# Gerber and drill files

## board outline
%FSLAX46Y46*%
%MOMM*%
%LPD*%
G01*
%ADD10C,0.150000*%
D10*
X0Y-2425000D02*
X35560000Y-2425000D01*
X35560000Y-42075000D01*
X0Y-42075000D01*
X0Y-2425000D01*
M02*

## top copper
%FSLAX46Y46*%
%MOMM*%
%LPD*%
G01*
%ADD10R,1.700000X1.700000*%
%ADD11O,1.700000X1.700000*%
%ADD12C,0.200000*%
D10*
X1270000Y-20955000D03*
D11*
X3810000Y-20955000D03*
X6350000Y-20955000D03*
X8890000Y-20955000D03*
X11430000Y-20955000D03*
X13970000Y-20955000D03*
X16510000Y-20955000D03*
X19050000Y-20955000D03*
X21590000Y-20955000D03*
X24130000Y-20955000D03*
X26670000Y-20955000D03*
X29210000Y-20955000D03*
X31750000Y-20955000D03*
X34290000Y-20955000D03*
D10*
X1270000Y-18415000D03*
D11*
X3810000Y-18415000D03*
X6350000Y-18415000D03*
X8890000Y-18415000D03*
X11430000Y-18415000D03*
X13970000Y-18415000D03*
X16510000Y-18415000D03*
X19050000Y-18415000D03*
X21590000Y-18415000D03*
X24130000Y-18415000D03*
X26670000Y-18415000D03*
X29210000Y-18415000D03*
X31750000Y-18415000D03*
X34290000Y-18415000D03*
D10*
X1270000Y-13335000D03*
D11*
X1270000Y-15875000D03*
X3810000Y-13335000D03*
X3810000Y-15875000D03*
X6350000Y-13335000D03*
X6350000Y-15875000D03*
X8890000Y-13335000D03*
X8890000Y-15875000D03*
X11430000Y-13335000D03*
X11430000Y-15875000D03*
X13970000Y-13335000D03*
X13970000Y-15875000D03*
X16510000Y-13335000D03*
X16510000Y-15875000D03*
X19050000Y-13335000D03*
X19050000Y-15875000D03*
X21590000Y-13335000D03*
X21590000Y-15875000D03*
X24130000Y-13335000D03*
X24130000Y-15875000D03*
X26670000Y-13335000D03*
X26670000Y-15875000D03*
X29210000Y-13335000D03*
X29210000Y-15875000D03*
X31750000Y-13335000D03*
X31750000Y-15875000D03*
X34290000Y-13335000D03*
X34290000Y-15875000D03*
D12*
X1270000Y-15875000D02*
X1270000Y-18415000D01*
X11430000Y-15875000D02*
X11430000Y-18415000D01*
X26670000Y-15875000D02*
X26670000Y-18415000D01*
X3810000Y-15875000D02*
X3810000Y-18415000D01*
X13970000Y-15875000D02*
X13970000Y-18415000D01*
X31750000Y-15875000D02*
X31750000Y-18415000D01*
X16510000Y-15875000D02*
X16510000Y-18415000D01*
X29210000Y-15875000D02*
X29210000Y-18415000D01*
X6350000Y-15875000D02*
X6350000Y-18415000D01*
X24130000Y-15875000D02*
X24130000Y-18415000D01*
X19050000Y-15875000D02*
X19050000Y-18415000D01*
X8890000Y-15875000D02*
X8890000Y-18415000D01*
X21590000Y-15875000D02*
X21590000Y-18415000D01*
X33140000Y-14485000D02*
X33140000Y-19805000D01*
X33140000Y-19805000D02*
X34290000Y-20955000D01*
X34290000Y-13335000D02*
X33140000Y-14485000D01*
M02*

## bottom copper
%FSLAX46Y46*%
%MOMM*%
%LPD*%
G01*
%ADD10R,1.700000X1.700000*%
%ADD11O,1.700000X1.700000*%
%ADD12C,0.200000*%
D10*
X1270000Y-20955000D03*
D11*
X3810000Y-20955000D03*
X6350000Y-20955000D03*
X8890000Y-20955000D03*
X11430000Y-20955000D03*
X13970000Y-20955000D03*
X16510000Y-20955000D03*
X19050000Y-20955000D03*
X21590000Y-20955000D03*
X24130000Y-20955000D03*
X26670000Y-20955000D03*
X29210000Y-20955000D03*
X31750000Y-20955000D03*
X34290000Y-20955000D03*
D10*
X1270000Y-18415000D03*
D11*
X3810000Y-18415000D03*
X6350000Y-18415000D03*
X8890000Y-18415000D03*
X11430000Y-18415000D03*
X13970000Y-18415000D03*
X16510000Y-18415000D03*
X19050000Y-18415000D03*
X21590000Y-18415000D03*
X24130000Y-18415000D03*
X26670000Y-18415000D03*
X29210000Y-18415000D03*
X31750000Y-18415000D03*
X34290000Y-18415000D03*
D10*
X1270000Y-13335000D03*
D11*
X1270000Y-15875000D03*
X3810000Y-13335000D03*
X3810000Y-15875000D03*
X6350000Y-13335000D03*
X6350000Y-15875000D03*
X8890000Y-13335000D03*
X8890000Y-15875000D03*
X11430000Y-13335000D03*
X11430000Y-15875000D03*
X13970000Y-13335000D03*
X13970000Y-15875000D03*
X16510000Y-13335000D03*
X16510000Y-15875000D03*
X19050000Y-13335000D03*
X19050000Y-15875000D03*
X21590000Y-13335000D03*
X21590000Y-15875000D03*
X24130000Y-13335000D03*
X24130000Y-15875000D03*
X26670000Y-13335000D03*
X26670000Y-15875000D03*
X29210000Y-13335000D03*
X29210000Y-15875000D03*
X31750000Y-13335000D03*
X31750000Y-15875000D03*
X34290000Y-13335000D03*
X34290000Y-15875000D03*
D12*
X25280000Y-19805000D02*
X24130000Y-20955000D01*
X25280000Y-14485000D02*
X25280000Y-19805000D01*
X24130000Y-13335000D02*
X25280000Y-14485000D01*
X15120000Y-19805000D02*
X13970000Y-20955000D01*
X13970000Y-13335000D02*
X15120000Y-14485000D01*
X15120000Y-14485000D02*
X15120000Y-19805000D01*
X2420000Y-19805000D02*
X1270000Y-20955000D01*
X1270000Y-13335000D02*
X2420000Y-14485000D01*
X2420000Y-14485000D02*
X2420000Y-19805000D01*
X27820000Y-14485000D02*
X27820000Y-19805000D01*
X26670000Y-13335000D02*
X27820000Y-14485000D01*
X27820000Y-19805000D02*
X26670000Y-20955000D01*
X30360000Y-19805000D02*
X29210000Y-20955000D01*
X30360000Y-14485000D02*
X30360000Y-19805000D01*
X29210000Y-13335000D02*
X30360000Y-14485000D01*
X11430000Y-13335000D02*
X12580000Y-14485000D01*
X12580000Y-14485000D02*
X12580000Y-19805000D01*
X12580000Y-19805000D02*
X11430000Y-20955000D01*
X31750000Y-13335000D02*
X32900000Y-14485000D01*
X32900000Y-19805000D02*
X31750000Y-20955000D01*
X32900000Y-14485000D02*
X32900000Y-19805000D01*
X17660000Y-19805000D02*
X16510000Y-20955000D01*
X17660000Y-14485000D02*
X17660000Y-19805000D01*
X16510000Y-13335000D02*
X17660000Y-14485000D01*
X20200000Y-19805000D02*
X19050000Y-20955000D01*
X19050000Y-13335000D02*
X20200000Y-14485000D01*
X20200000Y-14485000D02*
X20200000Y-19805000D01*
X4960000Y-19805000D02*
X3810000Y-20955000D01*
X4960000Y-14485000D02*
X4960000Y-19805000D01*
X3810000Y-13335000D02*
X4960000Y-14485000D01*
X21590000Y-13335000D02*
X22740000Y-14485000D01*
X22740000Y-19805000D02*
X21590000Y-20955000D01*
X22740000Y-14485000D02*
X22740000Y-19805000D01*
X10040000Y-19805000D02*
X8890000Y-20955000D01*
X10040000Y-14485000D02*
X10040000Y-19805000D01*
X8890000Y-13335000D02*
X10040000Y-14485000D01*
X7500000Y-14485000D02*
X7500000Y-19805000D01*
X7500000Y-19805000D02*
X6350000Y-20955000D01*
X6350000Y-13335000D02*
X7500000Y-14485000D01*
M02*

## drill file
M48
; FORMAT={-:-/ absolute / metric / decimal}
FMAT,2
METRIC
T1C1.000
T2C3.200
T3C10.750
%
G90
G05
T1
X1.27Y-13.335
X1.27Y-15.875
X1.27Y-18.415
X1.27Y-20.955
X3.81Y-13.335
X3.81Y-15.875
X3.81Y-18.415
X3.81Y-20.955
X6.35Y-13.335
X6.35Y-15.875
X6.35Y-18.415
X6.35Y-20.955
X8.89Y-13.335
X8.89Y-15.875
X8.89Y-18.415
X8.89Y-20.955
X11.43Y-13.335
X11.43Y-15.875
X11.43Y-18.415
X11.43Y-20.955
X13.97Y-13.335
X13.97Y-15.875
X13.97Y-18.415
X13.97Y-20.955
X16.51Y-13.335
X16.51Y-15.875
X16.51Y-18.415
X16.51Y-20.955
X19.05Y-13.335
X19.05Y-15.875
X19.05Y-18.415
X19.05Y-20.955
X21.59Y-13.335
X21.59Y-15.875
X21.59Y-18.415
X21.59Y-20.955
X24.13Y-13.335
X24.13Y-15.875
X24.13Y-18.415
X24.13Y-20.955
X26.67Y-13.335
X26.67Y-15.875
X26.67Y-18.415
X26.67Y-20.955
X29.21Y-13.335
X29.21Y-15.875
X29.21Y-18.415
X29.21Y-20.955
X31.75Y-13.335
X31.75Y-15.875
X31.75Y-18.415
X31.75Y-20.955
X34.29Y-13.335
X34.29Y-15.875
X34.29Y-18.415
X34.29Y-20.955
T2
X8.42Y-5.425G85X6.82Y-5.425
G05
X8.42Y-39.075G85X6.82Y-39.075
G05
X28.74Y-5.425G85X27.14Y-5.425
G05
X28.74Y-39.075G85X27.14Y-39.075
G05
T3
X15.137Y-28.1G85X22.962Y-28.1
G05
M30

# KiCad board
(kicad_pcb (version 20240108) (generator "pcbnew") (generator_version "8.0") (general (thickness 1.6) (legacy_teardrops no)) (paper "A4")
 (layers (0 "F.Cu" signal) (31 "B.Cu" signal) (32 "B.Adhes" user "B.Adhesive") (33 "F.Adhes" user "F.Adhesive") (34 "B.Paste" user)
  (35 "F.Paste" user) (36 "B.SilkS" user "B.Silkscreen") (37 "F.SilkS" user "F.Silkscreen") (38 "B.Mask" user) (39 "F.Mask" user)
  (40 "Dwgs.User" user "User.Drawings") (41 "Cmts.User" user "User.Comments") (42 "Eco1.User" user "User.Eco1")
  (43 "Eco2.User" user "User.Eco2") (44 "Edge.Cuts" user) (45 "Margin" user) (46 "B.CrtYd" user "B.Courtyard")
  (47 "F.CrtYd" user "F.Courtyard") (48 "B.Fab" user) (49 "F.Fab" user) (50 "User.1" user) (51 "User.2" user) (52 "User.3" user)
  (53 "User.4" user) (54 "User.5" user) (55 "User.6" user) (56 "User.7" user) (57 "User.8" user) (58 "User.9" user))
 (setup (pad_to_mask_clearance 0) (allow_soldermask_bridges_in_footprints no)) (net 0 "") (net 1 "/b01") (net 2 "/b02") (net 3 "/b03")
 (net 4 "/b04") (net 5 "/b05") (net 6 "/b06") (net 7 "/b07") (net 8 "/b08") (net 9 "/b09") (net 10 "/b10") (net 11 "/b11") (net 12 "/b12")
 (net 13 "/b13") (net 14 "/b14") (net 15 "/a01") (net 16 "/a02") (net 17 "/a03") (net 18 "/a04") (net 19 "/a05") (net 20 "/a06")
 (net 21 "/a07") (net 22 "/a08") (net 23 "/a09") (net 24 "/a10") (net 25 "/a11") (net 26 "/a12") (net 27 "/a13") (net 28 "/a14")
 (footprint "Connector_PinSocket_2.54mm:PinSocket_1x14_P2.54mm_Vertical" (layer "F.Cu") (at 1.27 20.955 90)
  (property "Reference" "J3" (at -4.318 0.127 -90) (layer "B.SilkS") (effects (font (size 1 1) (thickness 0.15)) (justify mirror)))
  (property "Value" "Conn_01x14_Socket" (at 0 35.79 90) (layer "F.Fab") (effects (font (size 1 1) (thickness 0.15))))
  (pad "1" thru_hole rect (at 0 0 90) (size 1.7 1.7) (drill 1) (layers "*.Cu" "*.Mask") (remove_unused_layers no) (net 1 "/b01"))
  (pad "2" thru_hole oval (at 0 2.54 90) (size 1.7 1.7) (drill 1) (layers "*.Cu" "*.Mask") (remove_unused_layers no) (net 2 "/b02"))
  (pad "3" thru_hole oval (at 0 5.08 90) (size 1.7 1.7) (drill 1) (layers "*.Cu" "*.Mask") (remove_unused_layers no) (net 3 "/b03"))
  (pad "4" thru_hole oval (at 0 7.62 90) (size 1.7 1.7) (drill 1) (layers "*.Cu" "*.Mask") (remove_unused_layers no) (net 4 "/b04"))
  (pad "5" thru_hole oval (at 0 10.16 90) (size 1.7 1.7) (drill 1) (layers "*.Cu" "*.Mask") (remove_unused_layers no) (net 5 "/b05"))
  (pad "6" thru_hole oval (at 0 12.7 90) (size 1.7 1.7) (drill 1) (layers "*.Cu" "*.Mask") (remove_unused_layers no) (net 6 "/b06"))
  (pad "7" thru_hole oval (at 0 15.24 90) (size 1.7 1.7) (drill 1) (layers "*.Cu" "*.Mask") (remove_unused_layers no) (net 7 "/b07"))
  (pad "8" thru_hole oval (at 0 17.78 90) (size 1.7 1.7) (drill 1) (layers "*.Cu" "*.Mask") (remove_unused_layers no) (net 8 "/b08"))
  (pad "9" thru_hole oval (at 0 20.32 90) (size 1.7 1.7) (drill 1) (layers "*.Cu" "*.Mask") (remove_unused_layers no) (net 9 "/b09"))
  (pad "10" thru_hole oval (at 0 22.86 90) (size 1.7 1.7) (drill 1) (layers "*.Cu" "*.Mask") (remove_unused_layers no) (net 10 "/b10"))
  (pad "11" thru_hole oval (at 0 25.4 90) (size 1.7 1.7) (drill 1) (layers "*.Cu" "*.Mask") (remove_unused_layers no) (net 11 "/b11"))
  (pad "12" thru_hole oval (at 0 27.94 90) (size 1.7 1.7) (drill 1) (layers "*.Cu" "*.Mask") (remove_unused_layers no) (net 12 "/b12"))
  (pad "13" thru_hole oval (at 0 30.48 90) (size 1.7 1.7) (drill 1) (layers "*.Cu" "*.Mask") (remove_unused_layers no) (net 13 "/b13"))
  (pad "14" thru_hole oval (at 0 33.02 90) (size 1.7 1.7) (drill 1) (layers "*.Cu" "*.Mask") (remove_unused_layers no) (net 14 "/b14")))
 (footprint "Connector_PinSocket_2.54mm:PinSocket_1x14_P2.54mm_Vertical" (layer "F.Cu") (at 1.27 18.415 90)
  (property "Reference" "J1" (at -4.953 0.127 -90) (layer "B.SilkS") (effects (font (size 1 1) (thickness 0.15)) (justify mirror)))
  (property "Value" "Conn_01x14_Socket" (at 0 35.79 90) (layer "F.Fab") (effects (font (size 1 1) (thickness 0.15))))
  (pad "1" thru_hole rect (at 0 0 90) (size 1.7 1.7) (drill 1) (layers "*.Cu" "*.Mask") (remove_unused_layers no) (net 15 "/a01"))
  (pad "2" thru_hole oval (at 0 2.54 90) (size 1.7 1.7) (drill 1) (layers "*.Cu" "*.Mask") (remove_unused_layers no) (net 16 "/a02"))
  (pad "3" thru_hole oval (at 0 5.08 90) (size 1.7 1.7) (drill 1) (layers "*.Cu" "*.Mask") (remove_unused_layers no) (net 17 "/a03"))
  (pad "4" thru_hole oval (at 0 7.62 90) (size 1.7 1.7) (drill 1) (layers "*.Cu" "*.Mask") (remove_unused_layers no) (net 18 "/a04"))
  (pad "5" thru_hole oval (at 0 10.16 90) (size 1.7 1.7) (drill 1) (layers "*.Cu" "*.Mask") (remove_unused_layers no) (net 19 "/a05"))
  (pad "6" thru_hole oval (at 0 12.7 90) (size 1.7 1.7) (drill 1) (layers "*.Cu" "*.Mask") (remove_unused_layers no) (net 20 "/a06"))
  (pad "7" thru_hole oval (at 0 15.24 90) (size 1.7 1.7) (drill 1) (layers "*.Cu" "*.Mask") (remove_unused_layers no) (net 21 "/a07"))
  (pad "8" thru_hole oval (at 0 17.78 90) (size 1.7 1.7) (drill 1) (layers "*.Cu" "*.Mask") (remove_unused_layers no) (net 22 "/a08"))
  (pad "9" thru_hole oval (at 0 20.32 90) (size 1.7 1.7) (drill 1) (layers "*.Cu" "*.Mask") (remove_unused_layers no) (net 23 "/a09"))
  (pad "10" thru_hole oval (at 0 22.86 90) (size 1.7 1.7) (drill 1) (layers "*.Cu" "*.Mask") (remove_unused_layers no) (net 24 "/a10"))
  (pad "11" thru_hole oval (at 0 25.4 90) (size 1.7 1.7) (drill 1) (layers "*.Cu" "*.Mask") (remove_unused_layers no) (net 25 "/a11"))
  (pad "12" thru_hole oval (at 0 27.94 90) (size 1.7 1.7) (drill 1) (layers "*.Cu" "*.Mask") (remove_unused_layers no) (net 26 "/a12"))
  (pad "13" thru_hole oval (at 0 30.48 90) (size 1.7 1.7) (drill 1) (layers "*.Cu" "*.Mask") (remove_unused_layers no) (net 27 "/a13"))
  (pad "14" thru_hole oval (at 0 33.02 90) (size 1.7 1.7) (drill 1) (layers "*.Cu" "*.Mask") (remove_unused_layers no) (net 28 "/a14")))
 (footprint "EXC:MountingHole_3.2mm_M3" (layer "F.Cu") (at 19.05 28.1)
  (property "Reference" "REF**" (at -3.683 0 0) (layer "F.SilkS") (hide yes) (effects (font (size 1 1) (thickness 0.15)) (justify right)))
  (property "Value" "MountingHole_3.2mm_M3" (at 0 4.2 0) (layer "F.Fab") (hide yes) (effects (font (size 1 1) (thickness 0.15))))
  (pad "" np_thru_hole oval (at 0 0) (size 18.575 10.75) (drill oval 18.575 10.75) (layers "F&B.Cu" "*.Mask")))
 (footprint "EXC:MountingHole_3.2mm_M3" (layer "B.Cu") (at 27.94 5.425 180)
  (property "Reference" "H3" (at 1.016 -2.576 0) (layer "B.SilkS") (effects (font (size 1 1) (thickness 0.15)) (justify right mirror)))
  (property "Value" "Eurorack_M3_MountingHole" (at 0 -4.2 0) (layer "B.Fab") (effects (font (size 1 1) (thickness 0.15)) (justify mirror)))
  (pad "" np_thru_hole oval (at 0 0 180) (size 4.8 3.2) (drill oval 4.8 3.2) (layers "F&B.Cu" "*.Mask")))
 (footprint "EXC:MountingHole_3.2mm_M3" (layer "B.Cu") (at 7.62 5.425 180)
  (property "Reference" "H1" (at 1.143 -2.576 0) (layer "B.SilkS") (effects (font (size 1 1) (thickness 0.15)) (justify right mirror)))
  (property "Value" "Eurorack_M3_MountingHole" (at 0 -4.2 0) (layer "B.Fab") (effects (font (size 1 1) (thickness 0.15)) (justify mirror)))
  (pad "" np_thru_hole oval (at 0 0 180) (size 4.8 3.2) (drill oval 4.8 3.2) (layers "F&B.Cu" "*.Mask")))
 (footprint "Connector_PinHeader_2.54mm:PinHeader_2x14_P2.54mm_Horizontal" (layer "B.Cu") (at 1.27 13.335 -90)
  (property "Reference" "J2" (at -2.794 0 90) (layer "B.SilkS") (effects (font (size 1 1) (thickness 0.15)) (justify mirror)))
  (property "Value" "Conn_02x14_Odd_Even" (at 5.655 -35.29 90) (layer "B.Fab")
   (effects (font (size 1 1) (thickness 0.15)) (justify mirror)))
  (pad "1" thru_hole rect (at 0 0 270) (size 1.7 1.7) (drill 1) (layers "*.Cu" "*.Mask") (remove_unused_layers no) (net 1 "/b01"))
  (pad "2" thru_hole oval (at 2.54 0 270) (size 1.7 1.7) (drill 1) (layers "*.Cu" "*.Mask") (remove_unused_layers no) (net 15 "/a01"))
  (pad "3" thru_hole oval (at 0 -2.54 270) (size 1.7 1.7) (drill 1) (layers "*.Cu" "*.Mask") (remove_unused_layers no) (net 2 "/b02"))
  (pad "4" thru_hole oval (at 2.54 -2.54 270) (size 1.7 1.7) (drill 1) (layers "*.Cu" "*.Mask") (remove_unused_layers no) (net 16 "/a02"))
  (pad "5" thru_hole oval (at 0 -5.08 270) (size 1.7 1.7) (drill 1) (layers "*.Cu" "*.Mask") (remove_unused_layers no) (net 3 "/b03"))
  (pad "6" thru_hole oval (at 2.54 -5.08 270) (size 1.7 1.7) (drill 1) (layers "*.Cu" "*.Mask") (remove_unused_layers no) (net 17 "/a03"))
  (pad "7" thru_hole oval (at 0 -7.62 270) (size 1.7 1.7) (drill 1) (layers "*.Cu" "*.Mask") (remove_unused_layers no) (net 4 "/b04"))
  (pad "8" thru_hole oval (at 2.54 -7.62 270) (size 1.7 1.7) (drill 1) (layers "*.Cu" "*.Mask") (remove_unused_layers no) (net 18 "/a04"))
  (pad "9" thru_hole oval (at 0 -10.16 270) (size 1.7 1.7) (drill 1) (layers "*.Cu" "*.Mask") (remove_unused_layers no) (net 5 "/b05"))
  (pad "10" thru_hole oval (at 2.54 -10.16 270) (size 1.7 1.7) (drill 1) (layers "*.Cu" "*.Mask") (remove_unused_layers no) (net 19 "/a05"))
  (pad "11" thru_hole oval (at 0 -12.7 270) (size 1.7 1.7) (drill 1) (layers "*.Cu" "*.Mask") (remove_unused_layers no) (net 6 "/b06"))
  (pad "12" thru_hole oval (at 2.54 -12.7 270) (size 1.7 1.7) (drill 1) (layers "*.Cu" "*.Mask") (remove_unused_layers no) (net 20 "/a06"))
  (pad "13" thru_hole oval (at 0 -15.24 270) (size 1.7 1.7) (drill 1) (layers "*.Cu" "*.Mask") (remove_unused_layers no) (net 7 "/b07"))
  (pad "14" thru_hole oval (at 2.54 -15.24 270) (size 1.7 1.7) (drill 1) (layers "*.Cu" "*.Mask") (remove_unused_layers no) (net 21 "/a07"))
  (pad "15" thru_hole oval (at 0 -17.78 270) (size 1.7 1.7) (drill 1) (layers "*.Cu" "*.Mask") (remove_unused_layers no) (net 8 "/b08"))
  (pad "16" thru_hole oval (at 2.54 -17.78 270) (size 1.7 1.7) (drill 1) (layers "*.Cu" "*.Mask") (remove_unused_layers no) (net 22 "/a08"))
  (pad "17" thru_hole oval (at 0 -20.32 270) (size 1.7 1.7) (drill 1) (layers "*.Cu" "*.Mask") (remove_unused_layers no) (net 9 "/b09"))
  (pad "18" thru_hole oval (at 2.54 -20.32 270) (size 1.7 1.7) (drill 1) (layers "*.Cu" "*.Mask") (remove_unused_layers no) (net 23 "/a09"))
  (pad "19" thru_hole oval (at 0 -22.86 270) (size 1.7 1.7) (drill 1) (layers "*.Cu" "*.Mask") (remove_unused_layers no) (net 10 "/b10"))
  (pad "20" thru_hole oval (at 2.54 -22.86 270) (size 1.7 1.7) (drill 1) (layers "*.Cu" "*.Mask") (remove_unused_layers no) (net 24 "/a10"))
  (pad "21" thru_hole oval (at 0 -25.4 270) (size 1.7 1.7) (drill 1) (layers "*.Cu" "*.Mask") (remove_unused_layers no) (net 11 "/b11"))
  (pad "22" thru_hole oval (at 2.54 -25.4 270) (size 1.7 1.7) (drill 1) (layers "*.Cu" "*.Mask") (remove_unused_layers no) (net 25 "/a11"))
  (pad "23" thru_hole oval (at 0 -27.94 270) (size 1.7 1.7) (drill 1) (layers "*.Cu" "*.Mask") (remove_unused_layers no) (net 12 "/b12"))
  (pad "24" thru_hole oval (at 2.54 -27.94 270) (size 1.7 1.7) (drill 1) (layers "*.Cu" "*.Mask") (remove_unused_layers no) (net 26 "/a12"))
  (pad "25" thru_hole oval (at 0 -30.48 270) (size 1.7 1.7) (drill 1) (layers "*.Cu" "*.Mask") (remove_unused_layers no) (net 13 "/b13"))
  (pad "26" thru_hole oval (at 2.54 -30.48 270) (size 1.7 1.7) (drill 1) (layers "*.Cu" "*.Mask") (remove_unused_layers no) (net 27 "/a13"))
  (pad "27" thru_hole oval (at 0 -33.02 270) (size 1.7 1.7) (drill 1) (layers "*.Cu" "*.Mask") (remove_unused_layers no) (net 14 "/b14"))
  (pad "28" thru_hole oval (at 2.54 -33.02 270) (size 1.7 1.7) (drill 1) (layers "*.Cu" "*.Mask") (remove_unused_layers no) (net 28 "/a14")))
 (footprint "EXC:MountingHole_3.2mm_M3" (layer "B.Cu") (at 27.94 39.075 180)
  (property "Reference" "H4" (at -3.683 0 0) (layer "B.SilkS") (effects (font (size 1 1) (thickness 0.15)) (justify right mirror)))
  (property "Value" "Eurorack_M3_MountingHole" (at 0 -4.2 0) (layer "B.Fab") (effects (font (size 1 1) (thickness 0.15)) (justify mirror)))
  (pad "" np_thru_hole oval (at 0 0 180) (size 4.8 3.2) (drill oval 4.8 3.2) (layers "F&B.Cu" "*.Mask")))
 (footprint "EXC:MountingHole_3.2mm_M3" (layer "B.Cu") (at 7.62 39.075 180)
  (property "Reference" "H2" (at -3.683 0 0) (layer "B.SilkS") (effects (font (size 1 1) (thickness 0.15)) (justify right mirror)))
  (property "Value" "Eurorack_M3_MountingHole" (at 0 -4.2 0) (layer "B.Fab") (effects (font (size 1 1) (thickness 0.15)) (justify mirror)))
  (pad "" np_thru_hole oval (at 0 0 180) (size 4.8 3.2) (drill oval 4.8 3.2) (layers "F&B.Cu" "*.Mask")))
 (gr_rect (start 0 2.425) (end 35.56 42.075) (stroke (width 0.15) (type default)) (fill none) (layer "Edge.Cuts"))
 (segment (start 1.27 15.875) (end 1.27 18.415) (width 0.2) (layer "F.Cu") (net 15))
 (segment (start 11.43 15.875) (end 11.43 18.415) (width 0.2) (layer "F.Cu") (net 19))
 (segment (start 26.67 15.875) (end 26.67 18.415) (width 0.2) (layer "F.Cu") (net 25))
 (segment (start 3.81 15.875) (end 3.81 18.415) (width 0.2) (layer "F.Cu") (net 16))
 (segment (start 13.97 15.875) (end 13.97 18.415) (width 0.2) (layer "F.Cu") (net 20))
 (segment (start 31.75 15.875) (end 31.75 18.415) (width 0.2) (layer "F.Cu") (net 27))
 (segment (start 16.51 15.875) (end 16.51 18.415) (width 0.2) (layer "F.Cu") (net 21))
 (segment (start 29.21 15.875) (end 29.21 18.415) (width 0.2) (layer "F.Cu") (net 26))
 (segment (start 6.35 15.875) (end 6.35 18.415) (width 0.2) (layer "F.Cu") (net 17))
 (segment (start 24.13 15.875) (end 24.13 18.415) (width 0.2) (layer "F.Cu") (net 24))
 (segment (start 19.05 15.875) (end 19.05 18.415) (width 0.2) (layer "F.Cu") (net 22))
 (segment (start 8.89 15.875) (end 8.89 18.415) (width 0.2) (layer "F.Cu") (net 18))
 (segment (start 21.59 15.875) (end 21.59 18.415) (width 0.2) (layer "F.Cu") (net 23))
 (segment (start 25.28 19.805) (end 24.13 20.955) (width 0.2) (layer "B.Cu") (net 10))
 (segment (start 25.28 14.485) (end 25.28 19.805) (width 0.2) (layer "B.Cu") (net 10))
 (segment (start 24.13 13.335) (end 25.28 14.485) (width 0.2) (layer "B.Cu") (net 10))
 (segment (start 15.12 19.805) (end 13.97 20.955) (width 0.2) (layer "B.Cu") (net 6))
 (segment (start 13.97 13.335) (end 15.12 14.485) (width 0.2) (layer "B.Cu") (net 6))
 (segment (start 15.12 14.485) (end 15.12 19.805) (width 0.2) (layer "B.Cu") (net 6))
 (segment (start 2.42 19.805) (end 1.27 20.955) (width 0.2) (layer "B.Cu") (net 1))
 (segment (start 1.27 13.335) (end 2.42 14.485) (width 0.2) (layer "B.Cu") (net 1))
 (segment (start 2.42 14.485) (end 2.42 19.805) (width 0.2) (layer "B.Cu") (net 1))
 (segment (start 27.82 14.485) (end 27.82 19.805) (width 0.2) (layer "B.Cu") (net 11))
 (segment (start 26.67 13.335) (end 27.82 14.485) (width 0.2) (layer "B.Cu") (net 11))
 (segment (start 27.82 19.805) (end 26.67 20.955) (width 0.2) (layer "B.Cu") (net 11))
 (segment (start 30.36 19.805) (end 29.21 20.955) (width 0.2) (layer "B.Cu") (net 12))
 (segment (start 30.36 14.485) (end 30.36 19.805) (width 0.2) (layer "B.Cu") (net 12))
 (segment (start 29.21 13.335) (end 30.36 14.485) (width 0.2) (layer "B.Cu") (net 12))
 (segment (start 11.43 13.335) (end 12.58 14.485) (width 0.2) (layer "B.Cu") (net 5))
 (segment (start 12.58 14.485) (end 12.58 19.805) (width 0.2) (layer "B.Cu") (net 5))
 (segment (start 12.58 19.805) (end 11.43 20.955) (width 0.2) (layer "B.Cu") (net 5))
 (segment (start 31.75 13.335) (end 32.9 14.485) (width 0.2) (layer "B.Cu") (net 13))
 (segment (start 32.9 19.805) (end 31.75 20.955) (width 0.2) (layer "B.Cu") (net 13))
 (segment (start 32.9 14.485) (end 32.9 19.805) (width 0.2) (layer "B.Cu") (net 13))
 (segment (start 17.66 19.805) (end 16.51 20.955) (width 0.2) (layer "B.Cu") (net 7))
 (segment (start 17.66 14.485) (end 17.66 19.805) (width 0.2) (layer "B.Cu") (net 7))
 (segment (start 16.51 13.335) (end 17.66 14.485) (width 0.2) (layer "B.Cu") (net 7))
 (segment (start 20.2 19.805) (end 19.05 20.955) (width 0.2) (layer "B.Cu") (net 8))
 (segment (start 19.05 13.335) (end 20.2 14.485) (width 0.2) (layer "B.Cu") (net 8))
 (segment (start 20.2 14.485) (end 20.2 19.805) (width 0.2) (layer "B.Cu") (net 8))
 (segment (start 4.96 19.805) (end 3.81 20.955) (width 0.2) (layer "B.Cu") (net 2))
 (segment (start 4.96 14.485) (end 4.96 19.805) (width 0.2) (layer "B.Cu") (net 2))
 (segment (start 3.81 13.335) (end 4.96 14.485) (width 0.2) (layer "B.Cu") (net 2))
 (segment (start 33.14 14.485) (end 33.14 19.805) (width 0.2) (layer "F.Cu") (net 14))
 (segment (start 33.14 19.805) (end 34.29 20.955) (width 0.2) (layer "F.Cu") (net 14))
 (segment (start 34.29 13.335) (end 33.14 14.485) (width 0.2) (layer "F.Cu") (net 14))
 (segment (start 21.59 13.335) (end 22.74 14.485) (width 0.2) (layer "B.Cu") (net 9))
 (segment (start 22.74 19.805) (end 21.59 20.955) (width 0.2) (layer "B.Cu") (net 9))
 (segment (start 22.74 14.485) (end 22.74 19.805) (width 0.2) (layer "B.Cu") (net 9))
 (segment (start 10.04 19.805) (end 8.89 20.955) (width 0.2) (layer "B.Cu") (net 4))
 (segment (start 10.04 14.485) (end 10.04 19.805) (width 0.2) (layer "B.Cu") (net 4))
 (segment (start 8.89 13.335) (end 10.04 14.485) (width 0.2) (layer "B.Cu") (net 4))
 (segment (start 7.5 14.485) (end 7.5 19.805) (width 0.2) (layer "B.Cu") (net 3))
 (segment (start 7.5 19.805) (end 6.35 20.955) (width 0.2) (layer "B.Cu") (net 3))
 (segment (start 6.35 13.335) (end 7.5 14.485) (width 0.2) (layer "B.Cu") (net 3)))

